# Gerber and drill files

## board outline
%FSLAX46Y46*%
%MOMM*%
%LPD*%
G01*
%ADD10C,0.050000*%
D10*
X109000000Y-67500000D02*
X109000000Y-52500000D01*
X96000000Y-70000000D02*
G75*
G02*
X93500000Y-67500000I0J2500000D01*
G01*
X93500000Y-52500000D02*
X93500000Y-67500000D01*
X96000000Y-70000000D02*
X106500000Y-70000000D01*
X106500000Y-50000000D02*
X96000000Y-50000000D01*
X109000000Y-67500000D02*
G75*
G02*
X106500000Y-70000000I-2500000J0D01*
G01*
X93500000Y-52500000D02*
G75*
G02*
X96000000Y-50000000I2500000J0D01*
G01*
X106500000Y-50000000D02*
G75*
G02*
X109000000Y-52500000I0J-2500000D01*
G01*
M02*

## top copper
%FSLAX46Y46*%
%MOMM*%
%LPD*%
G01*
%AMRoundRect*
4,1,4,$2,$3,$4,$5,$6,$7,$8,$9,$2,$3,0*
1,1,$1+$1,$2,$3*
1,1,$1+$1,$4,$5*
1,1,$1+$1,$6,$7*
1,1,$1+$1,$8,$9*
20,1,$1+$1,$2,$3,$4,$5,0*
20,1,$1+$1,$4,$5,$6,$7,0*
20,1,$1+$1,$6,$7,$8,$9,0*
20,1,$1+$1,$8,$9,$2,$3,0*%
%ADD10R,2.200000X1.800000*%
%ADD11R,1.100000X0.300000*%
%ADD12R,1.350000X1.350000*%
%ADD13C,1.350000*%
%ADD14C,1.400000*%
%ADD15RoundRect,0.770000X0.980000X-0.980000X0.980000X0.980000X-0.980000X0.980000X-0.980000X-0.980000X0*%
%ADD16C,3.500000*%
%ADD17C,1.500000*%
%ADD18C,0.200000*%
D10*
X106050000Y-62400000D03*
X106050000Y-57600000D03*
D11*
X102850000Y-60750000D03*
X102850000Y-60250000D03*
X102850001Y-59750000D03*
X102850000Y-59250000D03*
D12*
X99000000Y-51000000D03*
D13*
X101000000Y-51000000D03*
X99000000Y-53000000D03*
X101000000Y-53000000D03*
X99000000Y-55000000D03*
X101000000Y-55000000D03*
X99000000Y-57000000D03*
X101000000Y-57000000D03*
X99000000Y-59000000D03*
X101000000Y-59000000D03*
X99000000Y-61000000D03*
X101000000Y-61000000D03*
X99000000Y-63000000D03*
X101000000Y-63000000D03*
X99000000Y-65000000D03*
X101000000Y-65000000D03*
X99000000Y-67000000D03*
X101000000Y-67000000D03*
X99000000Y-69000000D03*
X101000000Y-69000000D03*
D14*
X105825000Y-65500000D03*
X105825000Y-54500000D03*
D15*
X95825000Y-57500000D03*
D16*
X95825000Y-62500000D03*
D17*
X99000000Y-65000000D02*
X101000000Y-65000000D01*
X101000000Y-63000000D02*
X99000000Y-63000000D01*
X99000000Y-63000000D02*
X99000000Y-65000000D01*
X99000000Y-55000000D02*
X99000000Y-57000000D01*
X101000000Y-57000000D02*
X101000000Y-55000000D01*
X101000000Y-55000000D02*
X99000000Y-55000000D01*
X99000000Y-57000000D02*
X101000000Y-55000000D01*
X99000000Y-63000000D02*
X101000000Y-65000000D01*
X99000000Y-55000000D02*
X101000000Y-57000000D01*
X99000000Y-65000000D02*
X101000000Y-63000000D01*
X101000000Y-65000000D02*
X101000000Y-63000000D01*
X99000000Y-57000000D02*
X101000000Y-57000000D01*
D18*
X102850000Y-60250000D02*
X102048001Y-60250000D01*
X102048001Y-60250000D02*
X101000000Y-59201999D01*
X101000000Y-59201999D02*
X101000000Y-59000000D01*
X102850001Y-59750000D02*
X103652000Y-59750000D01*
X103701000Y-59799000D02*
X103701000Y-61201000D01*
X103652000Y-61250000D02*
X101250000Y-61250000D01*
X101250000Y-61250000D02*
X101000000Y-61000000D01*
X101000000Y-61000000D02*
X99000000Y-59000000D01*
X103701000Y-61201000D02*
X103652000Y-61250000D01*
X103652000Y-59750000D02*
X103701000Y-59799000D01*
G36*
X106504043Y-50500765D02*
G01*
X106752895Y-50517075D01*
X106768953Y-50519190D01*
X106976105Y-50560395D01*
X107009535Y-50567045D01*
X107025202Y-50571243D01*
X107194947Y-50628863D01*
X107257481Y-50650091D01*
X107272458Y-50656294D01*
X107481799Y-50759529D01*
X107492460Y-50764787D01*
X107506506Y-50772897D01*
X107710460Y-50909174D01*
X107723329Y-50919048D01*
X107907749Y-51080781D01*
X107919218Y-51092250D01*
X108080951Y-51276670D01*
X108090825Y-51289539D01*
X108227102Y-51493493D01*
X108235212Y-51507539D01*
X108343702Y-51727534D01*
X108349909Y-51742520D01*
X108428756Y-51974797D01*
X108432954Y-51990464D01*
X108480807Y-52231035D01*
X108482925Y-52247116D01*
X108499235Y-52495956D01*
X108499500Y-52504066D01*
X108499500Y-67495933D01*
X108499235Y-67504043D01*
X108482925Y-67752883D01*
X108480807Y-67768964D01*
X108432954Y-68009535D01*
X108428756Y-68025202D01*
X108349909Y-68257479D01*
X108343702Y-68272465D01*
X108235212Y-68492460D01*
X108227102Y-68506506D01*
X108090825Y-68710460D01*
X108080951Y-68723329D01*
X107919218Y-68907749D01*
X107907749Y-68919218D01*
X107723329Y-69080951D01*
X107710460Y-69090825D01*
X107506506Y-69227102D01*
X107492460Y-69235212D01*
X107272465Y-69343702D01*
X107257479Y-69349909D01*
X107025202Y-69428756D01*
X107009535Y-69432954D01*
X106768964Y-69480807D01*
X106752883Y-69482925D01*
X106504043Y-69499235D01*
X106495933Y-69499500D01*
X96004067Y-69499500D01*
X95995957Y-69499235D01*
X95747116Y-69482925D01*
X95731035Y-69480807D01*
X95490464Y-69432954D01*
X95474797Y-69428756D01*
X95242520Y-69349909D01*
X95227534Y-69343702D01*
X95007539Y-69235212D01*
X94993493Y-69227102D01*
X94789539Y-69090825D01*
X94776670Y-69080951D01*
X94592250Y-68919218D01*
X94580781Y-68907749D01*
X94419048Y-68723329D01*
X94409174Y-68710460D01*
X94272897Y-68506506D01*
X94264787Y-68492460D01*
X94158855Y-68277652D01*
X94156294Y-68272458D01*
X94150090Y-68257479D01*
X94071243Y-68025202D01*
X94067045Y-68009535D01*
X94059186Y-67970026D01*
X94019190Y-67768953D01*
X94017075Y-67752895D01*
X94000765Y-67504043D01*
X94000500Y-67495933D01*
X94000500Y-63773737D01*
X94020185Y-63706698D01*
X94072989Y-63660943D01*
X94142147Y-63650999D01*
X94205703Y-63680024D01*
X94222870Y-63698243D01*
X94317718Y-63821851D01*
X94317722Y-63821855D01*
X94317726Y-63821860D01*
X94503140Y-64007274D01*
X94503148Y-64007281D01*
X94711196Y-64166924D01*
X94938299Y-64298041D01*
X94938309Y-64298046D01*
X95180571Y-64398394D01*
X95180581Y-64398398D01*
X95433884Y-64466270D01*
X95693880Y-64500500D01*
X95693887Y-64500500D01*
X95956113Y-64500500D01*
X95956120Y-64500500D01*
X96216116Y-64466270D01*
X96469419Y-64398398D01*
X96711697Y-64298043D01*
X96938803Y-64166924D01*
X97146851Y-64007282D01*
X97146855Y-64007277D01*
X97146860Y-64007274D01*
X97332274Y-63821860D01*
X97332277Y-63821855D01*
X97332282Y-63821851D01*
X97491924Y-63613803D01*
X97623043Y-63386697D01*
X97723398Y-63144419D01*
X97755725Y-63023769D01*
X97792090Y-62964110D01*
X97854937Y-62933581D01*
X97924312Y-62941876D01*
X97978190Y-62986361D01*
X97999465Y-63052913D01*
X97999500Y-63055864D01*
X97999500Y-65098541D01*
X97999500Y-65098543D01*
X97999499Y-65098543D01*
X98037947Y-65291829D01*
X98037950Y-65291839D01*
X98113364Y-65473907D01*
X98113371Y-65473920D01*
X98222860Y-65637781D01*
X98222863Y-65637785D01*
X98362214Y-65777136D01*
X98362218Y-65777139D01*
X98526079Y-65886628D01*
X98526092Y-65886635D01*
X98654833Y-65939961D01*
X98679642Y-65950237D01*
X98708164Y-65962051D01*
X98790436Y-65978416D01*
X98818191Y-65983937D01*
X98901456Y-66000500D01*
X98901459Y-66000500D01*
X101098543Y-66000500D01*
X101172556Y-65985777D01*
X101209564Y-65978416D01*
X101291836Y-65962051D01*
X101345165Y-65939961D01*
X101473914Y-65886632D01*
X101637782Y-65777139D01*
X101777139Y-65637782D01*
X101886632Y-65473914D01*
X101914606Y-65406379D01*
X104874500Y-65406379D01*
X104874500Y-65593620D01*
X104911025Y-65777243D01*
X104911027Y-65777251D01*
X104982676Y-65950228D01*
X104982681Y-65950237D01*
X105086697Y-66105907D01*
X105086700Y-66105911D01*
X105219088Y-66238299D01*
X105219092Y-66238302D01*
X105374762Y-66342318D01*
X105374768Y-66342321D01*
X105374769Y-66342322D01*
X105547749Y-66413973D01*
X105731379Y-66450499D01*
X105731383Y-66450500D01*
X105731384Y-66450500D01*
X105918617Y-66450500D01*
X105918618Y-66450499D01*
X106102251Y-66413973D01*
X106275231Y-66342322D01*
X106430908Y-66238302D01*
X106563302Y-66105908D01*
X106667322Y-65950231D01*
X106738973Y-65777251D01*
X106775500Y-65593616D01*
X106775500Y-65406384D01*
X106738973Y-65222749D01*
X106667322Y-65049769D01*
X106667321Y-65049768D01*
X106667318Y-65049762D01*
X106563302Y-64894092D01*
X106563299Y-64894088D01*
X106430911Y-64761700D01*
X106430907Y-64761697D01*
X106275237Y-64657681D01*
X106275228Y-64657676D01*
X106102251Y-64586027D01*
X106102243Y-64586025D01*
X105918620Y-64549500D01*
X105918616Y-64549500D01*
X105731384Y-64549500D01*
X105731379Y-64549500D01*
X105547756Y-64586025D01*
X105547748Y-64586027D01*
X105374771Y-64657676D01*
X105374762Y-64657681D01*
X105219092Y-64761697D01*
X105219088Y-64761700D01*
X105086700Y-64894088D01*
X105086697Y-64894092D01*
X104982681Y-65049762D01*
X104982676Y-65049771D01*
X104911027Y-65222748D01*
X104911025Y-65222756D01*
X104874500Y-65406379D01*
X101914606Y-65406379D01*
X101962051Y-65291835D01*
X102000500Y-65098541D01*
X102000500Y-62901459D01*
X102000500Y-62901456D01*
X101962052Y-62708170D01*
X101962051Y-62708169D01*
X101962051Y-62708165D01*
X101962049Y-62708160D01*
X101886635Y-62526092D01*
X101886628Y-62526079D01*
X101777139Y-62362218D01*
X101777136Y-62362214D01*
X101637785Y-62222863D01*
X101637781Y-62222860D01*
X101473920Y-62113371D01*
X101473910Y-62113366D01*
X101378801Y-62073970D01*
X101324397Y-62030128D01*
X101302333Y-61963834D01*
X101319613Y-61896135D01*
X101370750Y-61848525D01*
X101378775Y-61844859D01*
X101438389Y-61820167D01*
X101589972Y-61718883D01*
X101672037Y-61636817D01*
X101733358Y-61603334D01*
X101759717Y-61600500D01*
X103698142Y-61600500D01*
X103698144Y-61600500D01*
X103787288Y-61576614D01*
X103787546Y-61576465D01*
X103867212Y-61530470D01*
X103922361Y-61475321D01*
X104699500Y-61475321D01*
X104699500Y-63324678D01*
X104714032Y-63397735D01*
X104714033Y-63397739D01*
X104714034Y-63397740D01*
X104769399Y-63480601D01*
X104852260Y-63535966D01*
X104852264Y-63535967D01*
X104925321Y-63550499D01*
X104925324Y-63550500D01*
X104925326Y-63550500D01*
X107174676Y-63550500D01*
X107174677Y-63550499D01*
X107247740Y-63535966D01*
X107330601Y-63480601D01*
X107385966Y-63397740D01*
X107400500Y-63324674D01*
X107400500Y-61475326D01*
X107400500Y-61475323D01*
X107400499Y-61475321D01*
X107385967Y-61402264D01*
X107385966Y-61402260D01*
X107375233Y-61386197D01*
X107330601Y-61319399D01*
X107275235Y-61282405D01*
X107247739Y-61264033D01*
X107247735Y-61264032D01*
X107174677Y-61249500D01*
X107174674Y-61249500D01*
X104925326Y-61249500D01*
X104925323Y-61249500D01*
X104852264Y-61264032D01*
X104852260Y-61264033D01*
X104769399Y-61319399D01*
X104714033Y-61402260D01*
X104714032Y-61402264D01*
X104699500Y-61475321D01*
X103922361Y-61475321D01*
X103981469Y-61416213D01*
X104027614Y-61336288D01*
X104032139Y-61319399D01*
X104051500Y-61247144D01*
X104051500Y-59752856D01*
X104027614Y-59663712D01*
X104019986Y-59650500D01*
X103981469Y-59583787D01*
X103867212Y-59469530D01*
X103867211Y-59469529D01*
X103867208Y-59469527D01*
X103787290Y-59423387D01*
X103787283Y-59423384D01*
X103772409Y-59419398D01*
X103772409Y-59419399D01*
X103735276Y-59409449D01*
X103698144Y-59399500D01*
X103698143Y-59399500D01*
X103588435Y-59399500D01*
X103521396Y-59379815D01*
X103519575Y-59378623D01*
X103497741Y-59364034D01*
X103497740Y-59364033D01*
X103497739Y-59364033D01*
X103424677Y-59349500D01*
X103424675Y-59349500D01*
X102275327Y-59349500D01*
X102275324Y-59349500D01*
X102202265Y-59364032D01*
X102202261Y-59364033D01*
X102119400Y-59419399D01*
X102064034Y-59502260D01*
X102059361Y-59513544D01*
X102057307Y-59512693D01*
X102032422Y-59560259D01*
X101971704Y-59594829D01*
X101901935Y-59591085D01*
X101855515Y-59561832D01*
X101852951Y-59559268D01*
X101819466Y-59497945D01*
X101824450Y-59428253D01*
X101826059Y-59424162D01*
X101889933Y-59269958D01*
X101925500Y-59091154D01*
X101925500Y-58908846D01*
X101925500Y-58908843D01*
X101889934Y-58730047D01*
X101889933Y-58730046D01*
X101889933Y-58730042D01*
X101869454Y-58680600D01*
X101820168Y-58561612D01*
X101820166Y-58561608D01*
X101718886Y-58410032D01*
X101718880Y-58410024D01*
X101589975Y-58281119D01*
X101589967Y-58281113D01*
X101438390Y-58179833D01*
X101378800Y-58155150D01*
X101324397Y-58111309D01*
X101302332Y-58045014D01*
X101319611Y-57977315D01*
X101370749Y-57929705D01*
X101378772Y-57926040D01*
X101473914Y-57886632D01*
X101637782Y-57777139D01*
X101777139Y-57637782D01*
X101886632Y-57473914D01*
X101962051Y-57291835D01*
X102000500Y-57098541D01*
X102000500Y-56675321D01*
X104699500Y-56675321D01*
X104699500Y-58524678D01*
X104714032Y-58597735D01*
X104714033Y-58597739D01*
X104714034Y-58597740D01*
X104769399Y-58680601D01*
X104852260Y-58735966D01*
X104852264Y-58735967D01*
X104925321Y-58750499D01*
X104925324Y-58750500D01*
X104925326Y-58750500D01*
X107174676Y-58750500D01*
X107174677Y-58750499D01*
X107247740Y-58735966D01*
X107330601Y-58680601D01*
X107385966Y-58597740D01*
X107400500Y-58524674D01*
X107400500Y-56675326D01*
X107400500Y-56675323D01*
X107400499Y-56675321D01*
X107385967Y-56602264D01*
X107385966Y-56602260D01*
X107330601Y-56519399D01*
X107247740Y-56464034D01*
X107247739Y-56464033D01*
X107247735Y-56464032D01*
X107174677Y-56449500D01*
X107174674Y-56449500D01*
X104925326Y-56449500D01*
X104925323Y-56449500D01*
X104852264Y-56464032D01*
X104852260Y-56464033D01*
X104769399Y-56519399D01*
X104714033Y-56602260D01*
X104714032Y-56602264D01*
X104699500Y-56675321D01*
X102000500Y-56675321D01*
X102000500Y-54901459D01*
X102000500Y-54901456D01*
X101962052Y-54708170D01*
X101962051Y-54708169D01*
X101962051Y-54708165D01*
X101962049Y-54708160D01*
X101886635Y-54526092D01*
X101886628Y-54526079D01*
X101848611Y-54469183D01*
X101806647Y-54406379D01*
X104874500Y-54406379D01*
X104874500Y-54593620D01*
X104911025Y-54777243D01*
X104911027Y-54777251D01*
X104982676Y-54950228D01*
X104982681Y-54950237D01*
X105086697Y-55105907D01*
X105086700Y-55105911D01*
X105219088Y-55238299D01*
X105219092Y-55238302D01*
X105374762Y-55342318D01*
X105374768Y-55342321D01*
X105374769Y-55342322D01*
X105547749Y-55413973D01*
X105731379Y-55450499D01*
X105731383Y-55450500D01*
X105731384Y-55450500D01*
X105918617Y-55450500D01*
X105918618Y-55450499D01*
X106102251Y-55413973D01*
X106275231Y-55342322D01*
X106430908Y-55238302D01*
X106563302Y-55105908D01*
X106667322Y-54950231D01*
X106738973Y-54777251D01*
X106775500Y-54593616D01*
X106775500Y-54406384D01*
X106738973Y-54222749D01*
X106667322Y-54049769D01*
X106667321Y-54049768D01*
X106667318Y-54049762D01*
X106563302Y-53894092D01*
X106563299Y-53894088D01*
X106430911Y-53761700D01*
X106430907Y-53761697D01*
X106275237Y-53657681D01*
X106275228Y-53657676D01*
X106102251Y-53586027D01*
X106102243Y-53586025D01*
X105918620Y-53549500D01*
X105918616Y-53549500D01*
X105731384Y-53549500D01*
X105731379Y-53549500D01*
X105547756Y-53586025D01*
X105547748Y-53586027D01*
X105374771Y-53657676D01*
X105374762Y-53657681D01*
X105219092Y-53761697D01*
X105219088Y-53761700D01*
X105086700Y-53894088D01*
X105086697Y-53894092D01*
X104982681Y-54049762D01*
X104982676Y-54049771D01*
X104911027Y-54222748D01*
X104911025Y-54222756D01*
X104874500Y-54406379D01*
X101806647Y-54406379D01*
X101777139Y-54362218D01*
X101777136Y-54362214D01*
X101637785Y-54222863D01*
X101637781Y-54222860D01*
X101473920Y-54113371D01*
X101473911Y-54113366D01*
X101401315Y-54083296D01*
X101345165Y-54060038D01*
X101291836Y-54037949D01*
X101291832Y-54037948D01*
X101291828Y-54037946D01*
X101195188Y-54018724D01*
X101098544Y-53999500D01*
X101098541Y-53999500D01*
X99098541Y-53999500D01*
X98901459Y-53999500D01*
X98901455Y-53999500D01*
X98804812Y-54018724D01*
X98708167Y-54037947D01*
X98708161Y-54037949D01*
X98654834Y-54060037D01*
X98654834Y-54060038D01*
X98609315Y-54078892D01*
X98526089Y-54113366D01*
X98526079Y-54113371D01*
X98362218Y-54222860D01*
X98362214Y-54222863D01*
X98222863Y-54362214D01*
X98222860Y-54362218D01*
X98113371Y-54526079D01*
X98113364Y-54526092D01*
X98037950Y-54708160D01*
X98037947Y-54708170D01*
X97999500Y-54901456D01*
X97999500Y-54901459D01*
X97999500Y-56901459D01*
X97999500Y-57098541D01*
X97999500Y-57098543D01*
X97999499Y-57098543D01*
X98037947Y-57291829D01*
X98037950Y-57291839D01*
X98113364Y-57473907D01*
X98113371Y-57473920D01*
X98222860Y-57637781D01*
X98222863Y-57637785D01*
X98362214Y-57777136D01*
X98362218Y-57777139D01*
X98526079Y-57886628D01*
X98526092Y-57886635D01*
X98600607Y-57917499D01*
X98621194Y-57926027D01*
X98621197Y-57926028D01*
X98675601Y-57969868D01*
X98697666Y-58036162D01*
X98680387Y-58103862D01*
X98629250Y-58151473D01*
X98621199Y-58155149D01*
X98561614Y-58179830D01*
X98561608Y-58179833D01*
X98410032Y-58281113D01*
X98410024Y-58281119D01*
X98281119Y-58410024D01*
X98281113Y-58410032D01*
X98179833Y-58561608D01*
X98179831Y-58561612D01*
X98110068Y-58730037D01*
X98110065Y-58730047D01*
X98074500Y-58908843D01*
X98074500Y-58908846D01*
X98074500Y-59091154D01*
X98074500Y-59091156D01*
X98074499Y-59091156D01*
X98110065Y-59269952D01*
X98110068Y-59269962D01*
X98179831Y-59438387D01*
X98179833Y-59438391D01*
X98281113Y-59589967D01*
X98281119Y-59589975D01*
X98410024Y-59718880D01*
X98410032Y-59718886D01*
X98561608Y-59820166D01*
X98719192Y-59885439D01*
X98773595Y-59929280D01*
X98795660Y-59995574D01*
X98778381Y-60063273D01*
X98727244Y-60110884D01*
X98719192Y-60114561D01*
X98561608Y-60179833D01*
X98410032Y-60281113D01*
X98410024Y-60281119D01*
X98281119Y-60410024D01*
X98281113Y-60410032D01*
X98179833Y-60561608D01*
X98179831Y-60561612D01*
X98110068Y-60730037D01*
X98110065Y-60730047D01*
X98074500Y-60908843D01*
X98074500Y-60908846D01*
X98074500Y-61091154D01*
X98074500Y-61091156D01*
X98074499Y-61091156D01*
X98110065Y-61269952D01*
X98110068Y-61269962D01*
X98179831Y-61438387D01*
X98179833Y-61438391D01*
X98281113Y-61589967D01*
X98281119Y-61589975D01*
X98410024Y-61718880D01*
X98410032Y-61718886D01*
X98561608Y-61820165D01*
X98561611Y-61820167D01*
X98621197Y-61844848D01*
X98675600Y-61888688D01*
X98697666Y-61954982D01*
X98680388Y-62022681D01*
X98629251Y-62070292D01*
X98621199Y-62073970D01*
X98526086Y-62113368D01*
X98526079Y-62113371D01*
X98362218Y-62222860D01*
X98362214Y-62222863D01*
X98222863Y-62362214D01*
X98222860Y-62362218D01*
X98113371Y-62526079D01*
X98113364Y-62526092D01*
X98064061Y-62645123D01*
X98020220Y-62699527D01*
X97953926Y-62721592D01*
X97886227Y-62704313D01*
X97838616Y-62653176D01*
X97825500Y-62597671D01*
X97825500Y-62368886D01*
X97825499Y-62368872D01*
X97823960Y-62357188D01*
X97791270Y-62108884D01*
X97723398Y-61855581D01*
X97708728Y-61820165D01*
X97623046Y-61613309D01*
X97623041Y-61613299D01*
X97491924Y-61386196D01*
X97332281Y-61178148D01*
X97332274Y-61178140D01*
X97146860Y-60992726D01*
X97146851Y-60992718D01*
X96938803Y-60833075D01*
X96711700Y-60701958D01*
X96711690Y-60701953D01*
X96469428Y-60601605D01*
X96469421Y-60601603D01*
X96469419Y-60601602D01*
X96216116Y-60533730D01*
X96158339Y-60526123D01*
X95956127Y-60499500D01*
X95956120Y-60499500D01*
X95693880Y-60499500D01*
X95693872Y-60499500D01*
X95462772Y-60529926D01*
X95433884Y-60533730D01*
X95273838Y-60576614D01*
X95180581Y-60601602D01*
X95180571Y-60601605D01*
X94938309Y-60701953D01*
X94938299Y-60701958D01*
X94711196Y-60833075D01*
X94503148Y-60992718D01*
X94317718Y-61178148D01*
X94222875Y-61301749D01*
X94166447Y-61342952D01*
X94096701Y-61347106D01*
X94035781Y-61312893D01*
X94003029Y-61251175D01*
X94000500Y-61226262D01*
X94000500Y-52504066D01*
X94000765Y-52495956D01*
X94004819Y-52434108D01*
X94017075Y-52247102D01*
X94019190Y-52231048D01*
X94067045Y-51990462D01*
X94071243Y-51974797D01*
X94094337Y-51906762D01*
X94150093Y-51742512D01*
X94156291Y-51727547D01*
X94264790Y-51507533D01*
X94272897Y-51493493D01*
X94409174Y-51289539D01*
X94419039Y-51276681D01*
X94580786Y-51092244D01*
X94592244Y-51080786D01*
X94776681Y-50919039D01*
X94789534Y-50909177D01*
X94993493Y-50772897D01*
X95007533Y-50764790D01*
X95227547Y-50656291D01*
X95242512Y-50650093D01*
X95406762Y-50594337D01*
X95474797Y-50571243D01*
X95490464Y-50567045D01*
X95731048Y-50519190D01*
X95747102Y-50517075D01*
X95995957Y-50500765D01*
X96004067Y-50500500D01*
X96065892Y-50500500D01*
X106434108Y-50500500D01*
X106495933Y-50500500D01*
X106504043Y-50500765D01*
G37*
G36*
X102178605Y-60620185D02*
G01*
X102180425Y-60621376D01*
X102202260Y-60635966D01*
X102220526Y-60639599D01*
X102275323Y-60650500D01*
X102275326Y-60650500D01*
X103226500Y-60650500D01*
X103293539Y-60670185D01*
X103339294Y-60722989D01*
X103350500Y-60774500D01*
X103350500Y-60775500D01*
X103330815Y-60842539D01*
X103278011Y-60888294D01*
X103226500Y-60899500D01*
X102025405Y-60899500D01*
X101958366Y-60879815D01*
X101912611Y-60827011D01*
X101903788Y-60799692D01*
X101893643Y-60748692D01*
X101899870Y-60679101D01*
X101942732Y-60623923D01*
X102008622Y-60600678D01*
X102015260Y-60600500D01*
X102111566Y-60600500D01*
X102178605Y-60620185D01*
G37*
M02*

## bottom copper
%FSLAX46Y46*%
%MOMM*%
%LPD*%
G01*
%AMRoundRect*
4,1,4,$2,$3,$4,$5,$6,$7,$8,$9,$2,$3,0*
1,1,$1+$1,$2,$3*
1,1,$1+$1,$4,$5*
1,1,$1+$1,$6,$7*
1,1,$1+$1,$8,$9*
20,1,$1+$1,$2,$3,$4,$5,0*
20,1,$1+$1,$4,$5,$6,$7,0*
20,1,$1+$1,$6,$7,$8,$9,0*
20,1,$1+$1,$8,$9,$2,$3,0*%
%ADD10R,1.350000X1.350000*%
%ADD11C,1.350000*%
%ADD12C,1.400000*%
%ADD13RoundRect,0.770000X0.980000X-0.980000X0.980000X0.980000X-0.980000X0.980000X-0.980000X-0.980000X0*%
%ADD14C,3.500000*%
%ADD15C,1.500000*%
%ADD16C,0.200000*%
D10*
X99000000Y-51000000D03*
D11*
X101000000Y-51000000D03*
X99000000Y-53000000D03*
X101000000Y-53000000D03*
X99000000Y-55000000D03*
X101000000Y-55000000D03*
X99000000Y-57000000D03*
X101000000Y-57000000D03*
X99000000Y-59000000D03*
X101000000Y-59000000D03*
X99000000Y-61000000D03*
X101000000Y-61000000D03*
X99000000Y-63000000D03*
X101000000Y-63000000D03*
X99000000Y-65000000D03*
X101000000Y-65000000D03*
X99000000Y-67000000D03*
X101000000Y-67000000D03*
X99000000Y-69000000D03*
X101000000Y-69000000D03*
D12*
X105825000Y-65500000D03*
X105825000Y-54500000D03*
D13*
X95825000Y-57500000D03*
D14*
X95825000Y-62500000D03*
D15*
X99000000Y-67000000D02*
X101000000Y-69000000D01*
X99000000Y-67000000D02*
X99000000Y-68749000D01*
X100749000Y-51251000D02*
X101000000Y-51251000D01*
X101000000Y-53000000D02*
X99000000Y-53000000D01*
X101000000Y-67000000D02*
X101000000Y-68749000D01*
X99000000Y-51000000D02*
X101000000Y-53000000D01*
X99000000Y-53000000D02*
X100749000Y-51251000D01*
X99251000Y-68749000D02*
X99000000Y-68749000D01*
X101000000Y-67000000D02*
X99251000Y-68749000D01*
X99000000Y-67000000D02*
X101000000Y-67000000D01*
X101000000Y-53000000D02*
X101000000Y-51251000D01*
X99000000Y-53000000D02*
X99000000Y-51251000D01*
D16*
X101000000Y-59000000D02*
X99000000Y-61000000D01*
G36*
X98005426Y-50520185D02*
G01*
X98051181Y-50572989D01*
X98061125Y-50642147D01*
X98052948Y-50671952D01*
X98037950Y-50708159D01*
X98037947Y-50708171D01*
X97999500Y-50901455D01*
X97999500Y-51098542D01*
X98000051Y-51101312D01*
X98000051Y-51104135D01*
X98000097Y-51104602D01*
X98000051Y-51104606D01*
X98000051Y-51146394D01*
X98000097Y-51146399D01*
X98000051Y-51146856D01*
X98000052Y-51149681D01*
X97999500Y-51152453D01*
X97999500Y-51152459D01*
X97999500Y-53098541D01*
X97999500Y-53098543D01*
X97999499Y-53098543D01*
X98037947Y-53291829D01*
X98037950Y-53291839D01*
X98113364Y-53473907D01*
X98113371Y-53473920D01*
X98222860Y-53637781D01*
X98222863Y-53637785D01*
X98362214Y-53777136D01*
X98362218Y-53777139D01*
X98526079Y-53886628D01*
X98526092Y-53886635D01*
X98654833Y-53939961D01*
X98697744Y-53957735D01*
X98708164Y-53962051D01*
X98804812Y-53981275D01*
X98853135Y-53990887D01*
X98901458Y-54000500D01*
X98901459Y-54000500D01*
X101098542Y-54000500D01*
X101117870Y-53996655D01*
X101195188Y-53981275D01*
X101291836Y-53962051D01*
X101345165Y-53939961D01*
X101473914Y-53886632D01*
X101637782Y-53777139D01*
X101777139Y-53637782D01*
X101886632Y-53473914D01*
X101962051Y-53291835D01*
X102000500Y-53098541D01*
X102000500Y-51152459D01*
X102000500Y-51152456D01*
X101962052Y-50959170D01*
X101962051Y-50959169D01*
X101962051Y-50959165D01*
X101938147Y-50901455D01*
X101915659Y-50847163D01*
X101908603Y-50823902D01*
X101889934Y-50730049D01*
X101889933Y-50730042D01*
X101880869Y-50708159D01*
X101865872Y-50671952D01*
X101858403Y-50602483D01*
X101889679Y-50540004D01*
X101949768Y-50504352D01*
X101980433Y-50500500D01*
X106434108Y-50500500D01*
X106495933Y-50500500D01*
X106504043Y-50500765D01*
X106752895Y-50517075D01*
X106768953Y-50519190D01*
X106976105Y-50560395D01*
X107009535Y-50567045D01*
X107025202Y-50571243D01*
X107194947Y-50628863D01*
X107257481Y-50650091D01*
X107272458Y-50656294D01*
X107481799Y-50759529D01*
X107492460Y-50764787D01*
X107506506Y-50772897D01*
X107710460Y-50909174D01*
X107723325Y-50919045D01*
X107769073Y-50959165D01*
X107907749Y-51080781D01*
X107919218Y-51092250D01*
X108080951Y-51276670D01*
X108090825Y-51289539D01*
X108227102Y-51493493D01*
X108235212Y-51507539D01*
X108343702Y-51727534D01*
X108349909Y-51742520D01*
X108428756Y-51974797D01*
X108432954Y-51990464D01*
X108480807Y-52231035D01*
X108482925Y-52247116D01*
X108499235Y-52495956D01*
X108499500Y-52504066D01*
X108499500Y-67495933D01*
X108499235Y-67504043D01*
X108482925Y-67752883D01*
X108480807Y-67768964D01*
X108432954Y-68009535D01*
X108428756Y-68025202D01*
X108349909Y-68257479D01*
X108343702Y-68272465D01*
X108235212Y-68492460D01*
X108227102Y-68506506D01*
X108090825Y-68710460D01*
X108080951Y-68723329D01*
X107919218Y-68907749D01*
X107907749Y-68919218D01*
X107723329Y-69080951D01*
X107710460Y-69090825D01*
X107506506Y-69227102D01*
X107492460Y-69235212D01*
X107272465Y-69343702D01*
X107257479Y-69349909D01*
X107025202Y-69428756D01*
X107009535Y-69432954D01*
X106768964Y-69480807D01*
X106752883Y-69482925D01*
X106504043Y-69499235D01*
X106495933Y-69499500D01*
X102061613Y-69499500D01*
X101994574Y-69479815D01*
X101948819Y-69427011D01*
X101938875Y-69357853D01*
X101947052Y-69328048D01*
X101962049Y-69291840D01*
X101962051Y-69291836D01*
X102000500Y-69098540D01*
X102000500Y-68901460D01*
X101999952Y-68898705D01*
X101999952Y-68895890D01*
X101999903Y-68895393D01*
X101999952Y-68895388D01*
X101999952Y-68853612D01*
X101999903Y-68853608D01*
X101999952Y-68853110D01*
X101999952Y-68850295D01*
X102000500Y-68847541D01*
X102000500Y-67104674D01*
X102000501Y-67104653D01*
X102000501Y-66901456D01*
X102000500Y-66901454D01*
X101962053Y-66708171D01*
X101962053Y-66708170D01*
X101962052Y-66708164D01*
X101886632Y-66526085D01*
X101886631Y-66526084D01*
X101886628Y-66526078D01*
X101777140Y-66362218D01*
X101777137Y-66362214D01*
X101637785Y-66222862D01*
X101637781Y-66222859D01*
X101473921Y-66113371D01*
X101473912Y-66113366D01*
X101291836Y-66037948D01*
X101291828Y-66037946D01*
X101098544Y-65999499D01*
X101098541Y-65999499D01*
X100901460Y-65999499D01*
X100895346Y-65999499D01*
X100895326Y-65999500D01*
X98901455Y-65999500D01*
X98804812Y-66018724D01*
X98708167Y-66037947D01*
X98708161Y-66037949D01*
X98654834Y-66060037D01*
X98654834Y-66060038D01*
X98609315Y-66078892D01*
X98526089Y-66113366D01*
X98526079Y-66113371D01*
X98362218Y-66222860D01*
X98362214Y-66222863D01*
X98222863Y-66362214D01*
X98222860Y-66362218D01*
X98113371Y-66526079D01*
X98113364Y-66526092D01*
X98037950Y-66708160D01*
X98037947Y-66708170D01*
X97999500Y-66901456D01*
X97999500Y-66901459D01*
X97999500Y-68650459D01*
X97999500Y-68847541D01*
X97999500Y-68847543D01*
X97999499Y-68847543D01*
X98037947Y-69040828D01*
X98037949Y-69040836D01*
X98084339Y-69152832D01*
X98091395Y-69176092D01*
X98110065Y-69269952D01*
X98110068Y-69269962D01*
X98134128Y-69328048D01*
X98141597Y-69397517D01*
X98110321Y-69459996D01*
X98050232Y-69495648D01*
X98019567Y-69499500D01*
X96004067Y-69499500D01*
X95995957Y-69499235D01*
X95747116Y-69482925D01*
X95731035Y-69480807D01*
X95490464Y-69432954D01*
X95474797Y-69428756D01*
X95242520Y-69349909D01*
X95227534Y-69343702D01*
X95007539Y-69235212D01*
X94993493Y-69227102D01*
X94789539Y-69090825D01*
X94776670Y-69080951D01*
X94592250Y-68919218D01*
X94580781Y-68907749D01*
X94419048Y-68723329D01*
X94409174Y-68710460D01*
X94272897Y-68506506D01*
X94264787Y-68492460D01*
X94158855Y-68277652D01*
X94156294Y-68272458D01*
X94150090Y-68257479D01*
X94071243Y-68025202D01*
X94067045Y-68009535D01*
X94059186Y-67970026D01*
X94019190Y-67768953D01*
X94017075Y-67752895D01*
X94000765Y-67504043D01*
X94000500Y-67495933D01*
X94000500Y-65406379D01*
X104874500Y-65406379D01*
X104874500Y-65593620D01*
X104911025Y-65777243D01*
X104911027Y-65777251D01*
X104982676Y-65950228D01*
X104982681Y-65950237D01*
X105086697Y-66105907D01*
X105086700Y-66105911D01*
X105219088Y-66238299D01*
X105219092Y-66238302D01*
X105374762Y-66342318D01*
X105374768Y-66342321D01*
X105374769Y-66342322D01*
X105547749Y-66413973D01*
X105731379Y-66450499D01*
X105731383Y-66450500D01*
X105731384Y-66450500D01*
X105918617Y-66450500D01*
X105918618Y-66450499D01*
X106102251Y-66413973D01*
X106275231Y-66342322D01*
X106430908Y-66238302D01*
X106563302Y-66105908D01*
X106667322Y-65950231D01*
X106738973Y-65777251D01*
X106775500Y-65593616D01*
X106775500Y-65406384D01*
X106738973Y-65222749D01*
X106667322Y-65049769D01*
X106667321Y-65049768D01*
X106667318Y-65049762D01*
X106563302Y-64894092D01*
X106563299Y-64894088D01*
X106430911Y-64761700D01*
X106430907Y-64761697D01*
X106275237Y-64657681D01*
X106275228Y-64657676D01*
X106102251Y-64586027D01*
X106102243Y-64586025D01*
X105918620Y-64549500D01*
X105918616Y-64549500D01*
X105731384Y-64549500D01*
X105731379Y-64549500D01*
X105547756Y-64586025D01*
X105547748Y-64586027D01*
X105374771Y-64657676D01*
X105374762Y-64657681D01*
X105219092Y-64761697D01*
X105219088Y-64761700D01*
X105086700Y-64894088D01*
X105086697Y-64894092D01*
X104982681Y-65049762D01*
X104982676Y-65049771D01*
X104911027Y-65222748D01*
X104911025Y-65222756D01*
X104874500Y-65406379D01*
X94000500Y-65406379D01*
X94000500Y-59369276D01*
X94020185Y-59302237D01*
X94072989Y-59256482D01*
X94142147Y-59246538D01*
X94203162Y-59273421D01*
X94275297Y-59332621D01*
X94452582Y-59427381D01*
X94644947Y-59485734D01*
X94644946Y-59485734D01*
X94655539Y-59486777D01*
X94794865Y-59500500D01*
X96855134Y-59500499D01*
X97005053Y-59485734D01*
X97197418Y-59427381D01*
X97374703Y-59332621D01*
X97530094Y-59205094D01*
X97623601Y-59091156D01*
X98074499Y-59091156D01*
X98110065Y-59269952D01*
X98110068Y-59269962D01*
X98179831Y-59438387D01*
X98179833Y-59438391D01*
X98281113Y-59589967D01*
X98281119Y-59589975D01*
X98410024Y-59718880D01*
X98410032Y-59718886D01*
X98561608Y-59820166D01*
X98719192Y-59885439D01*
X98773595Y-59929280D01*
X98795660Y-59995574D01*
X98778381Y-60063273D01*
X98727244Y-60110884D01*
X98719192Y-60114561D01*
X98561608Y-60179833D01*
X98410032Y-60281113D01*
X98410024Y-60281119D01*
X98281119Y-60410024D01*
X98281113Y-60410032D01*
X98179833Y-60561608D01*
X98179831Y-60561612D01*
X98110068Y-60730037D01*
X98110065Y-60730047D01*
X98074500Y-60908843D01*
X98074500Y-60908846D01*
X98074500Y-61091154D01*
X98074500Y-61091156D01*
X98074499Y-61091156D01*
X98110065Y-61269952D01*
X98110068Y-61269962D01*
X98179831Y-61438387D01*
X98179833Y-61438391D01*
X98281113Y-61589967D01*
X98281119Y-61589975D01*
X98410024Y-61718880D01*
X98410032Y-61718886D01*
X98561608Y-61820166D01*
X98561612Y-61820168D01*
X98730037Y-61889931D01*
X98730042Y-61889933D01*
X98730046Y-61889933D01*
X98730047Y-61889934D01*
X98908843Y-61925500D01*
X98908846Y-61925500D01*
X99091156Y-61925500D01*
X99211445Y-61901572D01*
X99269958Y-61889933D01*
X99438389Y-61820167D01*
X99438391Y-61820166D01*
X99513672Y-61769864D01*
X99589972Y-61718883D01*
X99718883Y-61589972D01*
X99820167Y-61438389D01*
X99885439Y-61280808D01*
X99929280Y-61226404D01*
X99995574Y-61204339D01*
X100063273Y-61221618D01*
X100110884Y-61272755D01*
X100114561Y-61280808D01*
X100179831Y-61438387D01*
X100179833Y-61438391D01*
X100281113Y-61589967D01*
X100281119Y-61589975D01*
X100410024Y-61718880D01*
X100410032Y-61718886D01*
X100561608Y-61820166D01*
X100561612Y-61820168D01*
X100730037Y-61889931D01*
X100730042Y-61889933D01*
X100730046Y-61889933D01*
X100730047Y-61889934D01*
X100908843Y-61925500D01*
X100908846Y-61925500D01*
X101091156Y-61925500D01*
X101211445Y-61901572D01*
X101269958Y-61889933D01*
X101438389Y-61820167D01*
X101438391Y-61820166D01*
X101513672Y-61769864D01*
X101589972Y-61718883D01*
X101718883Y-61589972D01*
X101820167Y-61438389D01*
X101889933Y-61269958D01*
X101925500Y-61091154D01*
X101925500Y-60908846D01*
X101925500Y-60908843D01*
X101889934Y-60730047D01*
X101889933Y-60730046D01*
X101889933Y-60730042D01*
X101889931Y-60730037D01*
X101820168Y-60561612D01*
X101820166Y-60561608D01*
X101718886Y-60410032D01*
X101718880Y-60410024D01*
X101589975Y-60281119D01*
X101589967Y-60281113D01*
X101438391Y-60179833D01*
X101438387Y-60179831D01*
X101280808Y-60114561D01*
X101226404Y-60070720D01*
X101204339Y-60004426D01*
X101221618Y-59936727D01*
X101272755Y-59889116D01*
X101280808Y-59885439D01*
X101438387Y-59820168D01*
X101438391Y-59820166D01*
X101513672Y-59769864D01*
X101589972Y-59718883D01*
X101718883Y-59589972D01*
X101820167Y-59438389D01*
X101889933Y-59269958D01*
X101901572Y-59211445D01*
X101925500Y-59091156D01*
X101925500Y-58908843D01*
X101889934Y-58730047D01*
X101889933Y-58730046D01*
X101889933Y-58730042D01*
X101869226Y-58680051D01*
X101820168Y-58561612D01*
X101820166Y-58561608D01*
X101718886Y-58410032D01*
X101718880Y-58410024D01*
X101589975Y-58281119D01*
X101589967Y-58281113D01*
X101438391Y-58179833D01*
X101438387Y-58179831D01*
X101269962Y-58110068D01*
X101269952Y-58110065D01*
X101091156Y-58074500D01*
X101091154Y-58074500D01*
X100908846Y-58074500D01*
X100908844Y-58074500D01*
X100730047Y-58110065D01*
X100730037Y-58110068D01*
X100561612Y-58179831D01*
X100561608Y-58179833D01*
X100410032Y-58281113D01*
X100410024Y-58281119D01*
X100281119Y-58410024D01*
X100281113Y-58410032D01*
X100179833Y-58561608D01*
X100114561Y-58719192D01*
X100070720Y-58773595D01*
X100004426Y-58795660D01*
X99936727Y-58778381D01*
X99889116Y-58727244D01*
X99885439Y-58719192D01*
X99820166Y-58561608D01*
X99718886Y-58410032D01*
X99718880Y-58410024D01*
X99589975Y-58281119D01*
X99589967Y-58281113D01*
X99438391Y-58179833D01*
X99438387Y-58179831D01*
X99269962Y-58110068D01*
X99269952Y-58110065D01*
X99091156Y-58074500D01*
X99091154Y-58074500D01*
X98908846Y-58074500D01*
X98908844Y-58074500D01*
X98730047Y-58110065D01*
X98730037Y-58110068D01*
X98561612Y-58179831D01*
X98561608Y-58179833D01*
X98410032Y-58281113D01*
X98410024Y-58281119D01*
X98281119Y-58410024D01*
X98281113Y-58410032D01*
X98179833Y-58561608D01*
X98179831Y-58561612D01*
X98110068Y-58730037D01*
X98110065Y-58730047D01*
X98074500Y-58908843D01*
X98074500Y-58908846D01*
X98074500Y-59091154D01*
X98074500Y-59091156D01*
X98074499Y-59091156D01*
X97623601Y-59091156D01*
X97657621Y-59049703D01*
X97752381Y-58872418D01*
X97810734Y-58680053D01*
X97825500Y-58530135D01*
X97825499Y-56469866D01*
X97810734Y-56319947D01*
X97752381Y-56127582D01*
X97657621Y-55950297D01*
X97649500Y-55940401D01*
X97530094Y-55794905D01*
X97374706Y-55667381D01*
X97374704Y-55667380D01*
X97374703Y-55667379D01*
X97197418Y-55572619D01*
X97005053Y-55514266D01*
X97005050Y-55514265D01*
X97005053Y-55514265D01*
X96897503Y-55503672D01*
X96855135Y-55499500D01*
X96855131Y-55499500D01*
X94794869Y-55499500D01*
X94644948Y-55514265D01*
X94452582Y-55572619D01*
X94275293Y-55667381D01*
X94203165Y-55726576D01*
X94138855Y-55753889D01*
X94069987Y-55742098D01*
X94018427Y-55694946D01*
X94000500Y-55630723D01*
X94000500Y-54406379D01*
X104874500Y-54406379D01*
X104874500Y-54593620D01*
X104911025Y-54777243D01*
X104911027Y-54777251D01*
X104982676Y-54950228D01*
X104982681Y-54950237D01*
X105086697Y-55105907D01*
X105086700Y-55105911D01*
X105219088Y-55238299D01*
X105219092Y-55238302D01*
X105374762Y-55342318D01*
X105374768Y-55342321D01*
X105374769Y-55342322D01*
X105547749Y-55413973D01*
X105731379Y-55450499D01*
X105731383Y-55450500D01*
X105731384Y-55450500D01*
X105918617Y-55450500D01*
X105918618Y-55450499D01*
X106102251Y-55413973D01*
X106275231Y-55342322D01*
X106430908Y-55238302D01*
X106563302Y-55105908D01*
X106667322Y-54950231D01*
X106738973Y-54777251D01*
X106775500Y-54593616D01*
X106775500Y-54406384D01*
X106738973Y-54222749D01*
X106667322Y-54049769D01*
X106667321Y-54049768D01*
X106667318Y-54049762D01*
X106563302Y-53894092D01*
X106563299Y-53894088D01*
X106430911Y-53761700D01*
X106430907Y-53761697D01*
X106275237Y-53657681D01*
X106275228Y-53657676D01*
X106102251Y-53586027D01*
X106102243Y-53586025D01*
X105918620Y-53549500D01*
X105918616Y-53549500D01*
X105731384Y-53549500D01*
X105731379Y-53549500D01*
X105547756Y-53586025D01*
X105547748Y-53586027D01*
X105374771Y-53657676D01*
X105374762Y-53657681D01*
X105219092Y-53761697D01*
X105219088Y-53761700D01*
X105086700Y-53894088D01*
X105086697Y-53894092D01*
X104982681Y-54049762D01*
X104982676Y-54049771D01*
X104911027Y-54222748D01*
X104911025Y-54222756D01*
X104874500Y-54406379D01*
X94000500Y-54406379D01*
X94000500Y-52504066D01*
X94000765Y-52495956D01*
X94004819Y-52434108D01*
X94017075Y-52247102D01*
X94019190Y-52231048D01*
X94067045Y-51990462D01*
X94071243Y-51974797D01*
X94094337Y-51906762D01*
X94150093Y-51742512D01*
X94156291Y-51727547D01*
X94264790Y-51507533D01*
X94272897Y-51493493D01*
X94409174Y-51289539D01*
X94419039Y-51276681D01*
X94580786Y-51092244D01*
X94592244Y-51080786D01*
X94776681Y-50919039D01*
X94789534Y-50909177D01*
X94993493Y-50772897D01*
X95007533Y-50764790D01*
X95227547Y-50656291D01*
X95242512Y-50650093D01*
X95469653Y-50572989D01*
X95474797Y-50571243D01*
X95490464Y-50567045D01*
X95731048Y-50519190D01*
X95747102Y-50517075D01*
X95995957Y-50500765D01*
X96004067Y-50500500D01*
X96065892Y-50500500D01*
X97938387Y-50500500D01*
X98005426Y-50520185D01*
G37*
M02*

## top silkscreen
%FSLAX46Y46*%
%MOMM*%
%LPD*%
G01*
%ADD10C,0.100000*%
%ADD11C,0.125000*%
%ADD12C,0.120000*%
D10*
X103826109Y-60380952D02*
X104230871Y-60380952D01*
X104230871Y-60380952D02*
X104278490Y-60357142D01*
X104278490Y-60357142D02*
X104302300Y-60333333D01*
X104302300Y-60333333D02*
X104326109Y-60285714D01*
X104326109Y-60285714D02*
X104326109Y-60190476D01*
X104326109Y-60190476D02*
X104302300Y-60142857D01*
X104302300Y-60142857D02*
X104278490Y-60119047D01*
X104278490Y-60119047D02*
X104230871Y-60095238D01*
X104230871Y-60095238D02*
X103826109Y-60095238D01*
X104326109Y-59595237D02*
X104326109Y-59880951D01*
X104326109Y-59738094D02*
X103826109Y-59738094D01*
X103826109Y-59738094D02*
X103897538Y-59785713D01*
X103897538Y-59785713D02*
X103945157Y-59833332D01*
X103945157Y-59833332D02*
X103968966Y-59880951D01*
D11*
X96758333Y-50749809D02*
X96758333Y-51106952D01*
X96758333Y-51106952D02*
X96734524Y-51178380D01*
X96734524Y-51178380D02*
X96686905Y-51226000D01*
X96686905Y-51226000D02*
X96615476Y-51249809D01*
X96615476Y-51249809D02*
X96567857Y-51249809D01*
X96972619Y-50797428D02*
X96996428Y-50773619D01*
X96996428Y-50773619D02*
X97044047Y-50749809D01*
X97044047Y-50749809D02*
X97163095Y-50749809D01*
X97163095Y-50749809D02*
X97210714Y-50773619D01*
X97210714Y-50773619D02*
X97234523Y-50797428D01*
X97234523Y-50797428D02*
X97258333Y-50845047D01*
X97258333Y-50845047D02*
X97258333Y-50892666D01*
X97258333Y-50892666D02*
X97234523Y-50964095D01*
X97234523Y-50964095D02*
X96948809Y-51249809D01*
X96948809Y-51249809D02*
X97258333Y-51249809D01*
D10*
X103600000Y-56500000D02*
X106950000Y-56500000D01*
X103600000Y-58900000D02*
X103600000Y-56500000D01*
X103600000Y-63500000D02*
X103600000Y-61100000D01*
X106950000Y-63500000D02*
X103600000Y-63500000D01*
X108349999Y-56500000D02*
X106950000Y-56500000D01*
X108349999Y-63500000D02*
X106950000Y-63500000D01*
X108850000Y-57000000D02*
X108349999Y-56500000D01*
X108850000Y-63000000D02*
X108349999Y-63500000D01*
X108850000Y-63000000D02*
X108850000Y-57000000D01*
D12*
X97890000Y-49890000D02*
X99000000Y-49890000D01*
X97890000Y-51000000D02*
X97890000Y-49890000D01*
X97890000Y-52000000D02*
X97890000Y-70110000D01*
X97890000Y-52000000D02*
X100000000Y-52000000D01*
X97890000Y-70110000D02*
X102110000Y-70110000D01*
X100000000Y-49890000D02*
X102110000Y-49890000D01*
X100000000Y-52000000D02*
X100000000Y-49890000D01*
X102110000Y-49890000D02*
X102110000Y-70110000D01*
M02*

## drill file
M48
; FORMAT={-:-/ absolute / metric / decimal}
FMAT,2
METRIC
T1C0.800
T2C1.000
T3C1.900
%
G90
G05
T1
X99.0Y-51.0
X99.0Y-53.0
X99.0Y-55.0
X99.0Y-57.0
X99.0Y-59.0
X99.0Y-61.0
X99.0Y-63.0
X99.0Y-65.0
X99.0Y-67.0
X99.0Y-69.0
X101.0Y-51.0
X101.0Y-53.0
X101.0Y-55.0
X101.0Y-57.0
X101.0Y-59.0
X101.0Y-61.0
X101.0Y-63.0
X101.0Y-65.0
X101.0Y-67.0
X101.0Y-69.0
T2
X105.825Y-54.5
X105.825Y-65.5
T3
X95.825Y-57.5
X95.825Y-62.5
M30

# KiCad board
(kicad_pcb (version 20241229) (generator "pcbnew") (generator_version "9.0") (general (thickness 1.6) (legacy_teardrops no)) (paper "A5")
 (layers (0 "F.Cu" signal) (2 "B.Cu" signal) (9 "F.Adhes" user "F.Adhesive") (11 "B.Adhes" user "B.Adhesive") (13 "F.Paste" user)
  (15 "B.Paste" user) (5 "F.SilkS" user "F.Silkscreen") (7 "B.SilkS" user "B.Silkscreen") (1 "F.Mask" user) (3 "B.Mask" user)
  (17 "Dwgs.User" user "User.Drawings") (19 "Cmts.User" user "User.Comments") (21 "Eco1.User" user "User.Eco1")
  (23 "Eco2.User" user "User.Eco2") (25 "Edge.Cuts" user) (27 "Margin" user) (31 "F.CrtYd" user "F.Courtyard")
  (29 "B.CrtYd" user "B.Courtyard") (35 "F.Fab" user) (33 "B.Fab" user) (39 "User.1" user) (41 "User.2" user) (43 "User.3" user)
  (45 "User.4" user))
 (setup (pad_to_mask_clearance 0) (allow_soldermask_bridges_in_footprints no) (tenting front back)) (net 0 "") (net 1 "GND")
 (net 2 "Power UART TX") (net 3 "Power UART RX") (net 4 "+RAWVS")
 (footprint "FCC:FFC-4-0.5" (layer "F.Cu") (at 103.5 60 90)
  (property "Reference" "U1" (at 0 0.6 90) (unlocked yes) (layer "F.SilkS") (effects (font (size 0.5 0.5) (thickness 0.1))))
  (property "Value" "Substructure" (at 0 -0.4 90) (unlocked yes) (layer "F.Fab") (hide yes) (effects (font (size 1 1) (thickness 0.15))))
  (fp_line (start 3.5 0.1) (end 3.5 3.45) (stroke (width 0.1) (type default)) (layer "F.SilkS"))
  (fp_line (start 1.1 0.1) (end 3.5 0.1) (stroke (width 0.1) (type default)) (layer "F.SilkS"))
  (fp_line (start -3.5 0.1) (end -1.1 0.1) (stroke (width 0.1) (type default)) (layer "F.SilkS"))
  (fp_line (start -3.5 3.45) (end -3.5 0.1) (stroke (width 0.1) (type default)) (layer "F.SilkS"))
  (fp_line (start 3.5 4.849999) (end 3.5 3.45) (stroke (width 0.1) (type default)) (layer "F.SilkS"))
  (fp_line (start -3.5 4.849999) (end -3.5 3.45) (stroke (width 0.1) (type default)) (layer "F.SilkS"))
  (fp_line (start 3 5.35) (end 3.5 4.849999) (stroke (width 0.1) (type default)) (layer "F.SilkS"))
  (fp_line (start -3 5.35) (end -3.5 4.849999) (stroke (width 0.1) (type default)) (layer "F.SilkS"))
  (fp_line (start -3 5.35) (end 3 5.35) (stroke (width 0.1) (type default)) (layer "F.SilkS"))
  (pad "" smd rect (at -2.4 2.55 90) (size 1.8 2.2) (layers "F.Cu" "F.Mask" "F.Paste") (thermal_bridge_angle 45))
  (pad "" smd rect (at 2.4 2.55 90) (size 1.8 2.2) (layers "F.Cu" "F.Mask" "F.Paste") (thermal_bridge_angle 45))
  (pad "1" smd rect (at -0.75 -0.65 90) (size 0.3 1.1) (layers "F.Cu" "F.Mask" "F.Paste") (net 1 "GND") (thermal_bridge_angle 45))
  (pad "2" smd rect (at -0.25 -0.65 90) (size 0.3 1.1) (layers "F.Cu" "F.Mask" "F.Paste") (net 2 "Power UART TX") (thermal_bridge_angle 45))
  (pad "3" smd rect (at 0.25 -0.649999 90) (size 0.3 1.1) (layers "F.Cu" "F.Mask" "F.Paste") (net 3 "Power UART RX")
   (thermal_bridge_angle 45))
  (pad "4" smd rect (at 0.75 -0.65 90) (size 0.3 1.1) (layers "F.Cu" "F.Mask" "F.Paste") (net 1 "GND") (thermal_bridge_angle 45)))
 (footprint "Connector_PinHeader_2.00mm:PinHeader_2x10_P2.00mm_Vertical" (layer "F.Cu") (at 99 51)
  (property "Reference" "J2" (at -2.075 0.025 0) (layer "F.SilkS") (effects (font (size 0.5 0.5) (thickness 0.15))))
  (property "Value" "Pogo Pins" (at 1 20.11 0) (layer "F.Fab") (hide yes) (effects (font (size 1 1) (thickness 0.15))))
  (fp_line (start -1.11 -1.11) (end 0 -1.11) (stroke (width 0.12) (type solid)) (layer "F.SilkS"))
  (fp_line (start -1.11 0) (end -1.11 -1.11) (stroke (width 0.12) (type solid)) (layer "F.SilkS"))
  (fp_line (start -1.11 1) (end -1.11 19.11) (stroke (width 0.12) (type solid)) (layer "F.SilkS"))
  (fp_line (start -1.11 1) (end 1 1) (stroke (width 0.12) (type solid)) (layer "F.SilkS"))
  (fp_line (start -1.11 19.11) (end 3.11 19.11) (stroke (width 0.12) (type solid)) (layer "F.SilkS"))
  (fp_line (start 1 -1.11) (end 3.11 -1.11) (stroke (width 0.12) (type solid)) (layer "F.SilkS"))
  (fp_line (start 1 1) (end 1 -1.11) (stroke (width 0.12) (type solid)) (layer "F.SilkS"))
  (fp_line (start 3.11 -1.11) (end 3.11 19.11) (stroke (width 0.12) (type solid)) (layer "F.SilkS"))
  (pad "1" thru_hole rect (at 0 0) (size 1.35 1.35) (drill 0.8) (layers "*.Cu" "*.Mask") (remove_unused_layers no) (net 1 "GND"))
  (pad "2" thru_hole circle (at 2 0) (size 1.35 1.35) (drill 0.8) (layers "*.Cu" "*.Mask") (remove_unused_layers no) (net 1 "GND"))
  (pad "3" thru_hole circle (at 0 2) (size 1.35 1.35) (drill 0.8) (layers "*.Cu" "*.Mask") (remove_unused_layers no) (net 1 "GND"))
  (pad "4" thru_hole circle (at 2 2) (size 1.35 1.35) (drill 0.8) (layers "*.Cu" "*.Mask") (remove_unused_layers no) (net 1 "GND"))
  (pad "5" thru_hole circle (at 0 4) (size 1.35 1.35) (drill 0.8) (layers "*.Cu" "*.Mask") (remove_unused_layers no) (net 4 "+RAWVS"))
  (pad "6" thru_hole circle (at 2 4) (size 1.35 1.35) (drill 0.8) (layers "*.Cu" "*.Mask") (remove_unused_layers no) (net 4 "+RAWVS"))
  (pad "7" thru_hole circle (at 0 6) (size 1.35 1.35) (drill 0.8) (layers "*.Cu" "*.Mask") (remove_unused_layers no) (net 4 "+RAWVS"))
  (pad "8" thru_hole circle (at 2 6) (size 1.35 1.35) (drill 0.8) (layers "*.Cu" "*.Mask") (remove_unused_layers no) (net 4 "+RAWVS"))
  (pad "9" thru_hole circle (at 0 8) (size 1.35 1.35) (drill 0.8) (layers "*.Cu" "*.Mask") (remove_unused_layers no) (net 3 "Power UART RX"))
  (pad "10" thru_hole circle (at 2 8) (size 1.35 1.35) (drill 0.8) (layers "*.Cu" "*.Mask") (remove_unused_layers no)
   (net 2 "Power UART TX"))
  (pad "11" thru_hole circle (at 0 10) (size 1.35 1.35) (drill 0.8) (layers "*.Cu" "*.Mask") (remove_unused_layers no)
   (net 2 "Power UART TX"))
  (pad "12" thru_hole circle (at 2 10) (size 1.35 1.35) (drill 0.8) (layers "*.Cu" "*.Mask") (remove_unused_layers no)
   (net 3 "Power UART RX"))
  (pad "13" thru_hole circle (at 0 12) (size 1.35 1.35) (drill 0.8) (layers "*.Cu" "*.Mask") (remove_unused_layers no) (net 4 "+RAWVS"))
  (pad "14" thru_hole circle (at 2 12) (size 1.35 1.35) (drill 0.8) (layers "*.Cu" "*.Mask") (remove_unused_layers no) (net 4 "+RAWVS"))
  (pad "15" thru_hole circle (at 0 14) (size 1.35 1.35) (drill 0.8) (layers "*.Cu" "*.Mask") (remove_unused_layers no) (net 4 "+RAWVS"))
  (pad "16" thru_hole circle (at 2 14) (size 1.35 1.35) (drill 0.8) (layers "*.Cu" "*.Mask") (remove_unused_layers no) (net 4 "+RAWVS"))
  (pad "17" thru_hole circle (at 0 16) (size 1.35 1.35) (drill 0.8) (layers "*.Cu" "*.Mask") (remove_unused_layers no) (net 1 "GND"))
  (pad "18" thru_hole circle (at 2 16) (size 1.35 1.35) (drill 0.8) (layers "*.Cu" "*.Mask") (remove_unused_layers no) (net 1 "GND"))
  (pad "19" thru_hole circle (at 0 18) (size 1.35 1.35) (drill 0.8) (layers "*.Cu" "*.Mask") (remove_unused_layers no) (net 1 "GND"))
  (pad "20" thru_hole circle (at 2 18) (size 1.35 1.35) (drill 0.8) (layers "*.Cu" "*.Mask") (remove_unused_layers no) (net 1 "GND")))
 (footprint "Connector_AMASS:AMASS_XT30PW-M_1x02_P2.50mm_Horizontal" (layer "B.Cu") (at 95.825 57.5 90)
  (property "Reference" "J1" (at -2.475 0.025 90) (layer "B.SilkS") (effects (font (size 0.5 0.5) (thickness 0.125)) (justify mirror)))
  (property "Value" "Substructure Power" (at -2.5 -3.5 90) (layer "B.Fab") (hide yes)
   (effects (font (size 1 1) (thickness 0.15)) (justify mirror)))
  (pad "" thru_hole circle (at -8 10 90) (size 1.4 1.4) (drill 1) (layers "*.Cu" "*.Mask") (remove_unused_layers no))
  (pad "" thru_hole circle (at 3 10 90) (size 1.4 1.4) (drill 1) (layers "*.Cu" "*.Mask") (remove_unused_layers no))
  (pad "1" thru_hole roundrect (at 0 0 90) (size 3.5 3.5) (drill 1.9) (layers "*.Cu" "*.Mask") (remove_unused_layers no)
   (roundrect_rratio 0.22) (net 1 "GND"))
  (pad "2" thru_hole circle (at -5 0 90) (size 3.5 3.5) (drill 1.9) (layers "*.Cu" "*.Mask") (remove_unused_layers no) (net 4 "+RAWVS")))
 (gr_line (start 109 67.5) (end 109 52.5) (stroke (width 0.05) (type default)) (layer "Edge.Cuts"))
 (gr_arc (start 96 70) (mid 94.232233 69.267767) (end 93.5 67.5) (stroke (width 0.05) (type default)) (layer "Edge.Cuts"))
 (gr_line (start 93.5 52.5) (end 93.5 67.5) (stroke (width 0.05) (type default)) (layer "Edge.Cuts"))
 (gr_line (start 96 70) (end 106.5 70) (stroke (width 0.05) (type default)) (layer "Edge.Cuts"))
 (gr_line (start 106.5 50) (end 96 50) (stroke (width 0.05) (type default)) (layer "Edge.Cuts"))
 (gr_arc (start 109 67.5) (mid 108.267767 69.267767) (end 106.5 70) (stroke (width 0.05) (type default)) (layer "Edge.Cuts"))
 (gr_arc (start 93.5 52.5) (mid 94.232233 50.732233) (end 96 50) (stroke (width 0.05) (type default)) (layer "Edge.Cuts"))
 (gr_arc (start 106.5 50) (mid 108.267767 50.732233) (end 109 52.5) (stroke (width 0.05) (type default)) (layer "Edge.Cuts"))
 (segment (start 99 65) (end 101 65) (width 1.5) (layer "F.Cu") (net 4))
 (segment (start 101 63) (end 99 63) (width 1.5) (layer "F.Cu") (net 4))
 (segment (start 99 63) (end 99 65) (width 1.5) (layer "F.Cu") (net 4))
 (segment (start 99 55) (end 99 57) (width 1.5) (layer "F.Cu") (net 4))
 (segment (start 101 57) (end 101 55) (width 1.5) (layer "F.Cu") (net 4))
 (segment (start 101 55) (end 99 55) (width 1.5) (layer "F.Cu") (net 4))
 (segment (start 99 57) (end 101 55) (width 1.5) (layer "F.Cu") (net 4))
 (segment (start 99 63) (end 101 65) (width 1.5) (layer "F.Cu") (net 4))
 (segment (start 99 55) (end 101 57) (width 1.5) (layer "F.Cu") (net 4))
 (segment (start 99 65) (end 101 63) (width 1.5) (layer "F.Cu") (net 4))
 (segment (start 101 65) (end 101 63) (width 1.5) (layer "F.Cu") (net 4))
 (segment (start 99 57) (end 101 57) (width 1.5) (layer "F.Cu") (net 4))
 (segment (start 99 67) (end 101 69) (width 1.5) (layer "B.Cu") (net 1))
 (segment (start 99 67) (end 99 68.749) (width 1.5) (layer "B.Cu") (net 1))
 (segment (start 100.749 51.251) (end 101 51.251) (width 1.5) (layer "B.Cu") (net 1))
 (segment (start 101 53) (end 99 53) (width 1.5) (layer "B.Cu") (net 1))
 (segment (start 101 67) (end 101 68.749) (width 1.5) (layer "B.Cu") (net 1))
 (segment (start 99 51) (end 101 53) (width 1.5) (layer "B.Cu") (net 1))
 (segment (start 99 53) (end 100.749 51.251) (width 1.5) (layer "B.Cu") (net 1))
 (segment (start 99.251 68.749) (end 99 68.749) (width 1.5) (layer "B.Cu") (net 1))
 (segment (start 101 67) (end 99.251 68.749) (width 1.5) (layer "B.Cu") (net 1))
 (segment (start 99 67) (end 101 67) (width 1.5) (layer "B.Cu") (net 1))
 (segment (start 101 53) (end 101 51.251) (width 1.5) (layer "B.Cu") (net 1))
 (segment (start 99 53) (end 99 51.251) (width 1.5) (layer "B.Cu") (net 1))
 (segment (start 102.85 60.25) (end 102.048001 60.25) (width 0.2) (layer "F.Cu") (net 2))
 (segment (start 102.048001 60.25) (end 101 59.201999) (width 0.2) (layer "F.Cu") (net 2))
 (segment (start 101 59.201999) (end 101 59) (width 0.2) (layer "F.Cu") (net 2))
 (segment (start 101 59) (end 99 61) (width 0.2) (layer "B.Cu") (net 2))
 (segment (start 102.850001 59.75) (end 103.652 59.75) (width 0.2) (layer "F.Cu") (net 3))
 (segment (start 103.701 59.799) (end 103.701 61.201) (width 0.2) (layer "F.Cu") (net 3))
 (segment (start 103.652 61.25) (end 101.25 61.25) (width 0.2) (layer "F.Cu") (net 3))
 (segment (start 101.25 61.25) (end 101 61) (width 0.2) (layer "F.Cu") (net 3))
 (segment (start 101 61) (end 99 59) (width 0.2) (layer "F.Cu") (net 3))
 (segment (start 103.701 61.201) (end 103.652 61.25) (width 0.2) (layer "F.Cu") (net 3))
 (segment (start 103.652 59.75) (end 103.701 59.799) (width 0.2) (layer "F.Cu") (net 3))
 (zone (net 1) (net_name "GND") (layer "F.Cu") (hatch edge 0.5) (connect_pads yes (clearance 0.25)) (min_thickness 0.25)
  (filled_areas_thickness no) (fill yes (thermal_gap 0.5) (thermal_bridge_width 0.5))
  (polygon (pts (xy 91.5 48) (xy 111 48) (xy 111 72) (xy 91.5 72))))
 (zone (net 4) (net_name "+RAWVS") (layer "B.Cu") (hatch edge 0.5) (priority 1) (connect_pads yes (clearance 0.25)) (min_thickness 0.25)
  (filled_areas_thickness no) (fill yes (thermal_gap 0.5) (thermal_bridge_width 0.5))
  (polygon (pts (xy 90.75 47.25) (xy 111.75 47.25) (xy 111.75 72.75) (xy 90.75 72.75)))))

